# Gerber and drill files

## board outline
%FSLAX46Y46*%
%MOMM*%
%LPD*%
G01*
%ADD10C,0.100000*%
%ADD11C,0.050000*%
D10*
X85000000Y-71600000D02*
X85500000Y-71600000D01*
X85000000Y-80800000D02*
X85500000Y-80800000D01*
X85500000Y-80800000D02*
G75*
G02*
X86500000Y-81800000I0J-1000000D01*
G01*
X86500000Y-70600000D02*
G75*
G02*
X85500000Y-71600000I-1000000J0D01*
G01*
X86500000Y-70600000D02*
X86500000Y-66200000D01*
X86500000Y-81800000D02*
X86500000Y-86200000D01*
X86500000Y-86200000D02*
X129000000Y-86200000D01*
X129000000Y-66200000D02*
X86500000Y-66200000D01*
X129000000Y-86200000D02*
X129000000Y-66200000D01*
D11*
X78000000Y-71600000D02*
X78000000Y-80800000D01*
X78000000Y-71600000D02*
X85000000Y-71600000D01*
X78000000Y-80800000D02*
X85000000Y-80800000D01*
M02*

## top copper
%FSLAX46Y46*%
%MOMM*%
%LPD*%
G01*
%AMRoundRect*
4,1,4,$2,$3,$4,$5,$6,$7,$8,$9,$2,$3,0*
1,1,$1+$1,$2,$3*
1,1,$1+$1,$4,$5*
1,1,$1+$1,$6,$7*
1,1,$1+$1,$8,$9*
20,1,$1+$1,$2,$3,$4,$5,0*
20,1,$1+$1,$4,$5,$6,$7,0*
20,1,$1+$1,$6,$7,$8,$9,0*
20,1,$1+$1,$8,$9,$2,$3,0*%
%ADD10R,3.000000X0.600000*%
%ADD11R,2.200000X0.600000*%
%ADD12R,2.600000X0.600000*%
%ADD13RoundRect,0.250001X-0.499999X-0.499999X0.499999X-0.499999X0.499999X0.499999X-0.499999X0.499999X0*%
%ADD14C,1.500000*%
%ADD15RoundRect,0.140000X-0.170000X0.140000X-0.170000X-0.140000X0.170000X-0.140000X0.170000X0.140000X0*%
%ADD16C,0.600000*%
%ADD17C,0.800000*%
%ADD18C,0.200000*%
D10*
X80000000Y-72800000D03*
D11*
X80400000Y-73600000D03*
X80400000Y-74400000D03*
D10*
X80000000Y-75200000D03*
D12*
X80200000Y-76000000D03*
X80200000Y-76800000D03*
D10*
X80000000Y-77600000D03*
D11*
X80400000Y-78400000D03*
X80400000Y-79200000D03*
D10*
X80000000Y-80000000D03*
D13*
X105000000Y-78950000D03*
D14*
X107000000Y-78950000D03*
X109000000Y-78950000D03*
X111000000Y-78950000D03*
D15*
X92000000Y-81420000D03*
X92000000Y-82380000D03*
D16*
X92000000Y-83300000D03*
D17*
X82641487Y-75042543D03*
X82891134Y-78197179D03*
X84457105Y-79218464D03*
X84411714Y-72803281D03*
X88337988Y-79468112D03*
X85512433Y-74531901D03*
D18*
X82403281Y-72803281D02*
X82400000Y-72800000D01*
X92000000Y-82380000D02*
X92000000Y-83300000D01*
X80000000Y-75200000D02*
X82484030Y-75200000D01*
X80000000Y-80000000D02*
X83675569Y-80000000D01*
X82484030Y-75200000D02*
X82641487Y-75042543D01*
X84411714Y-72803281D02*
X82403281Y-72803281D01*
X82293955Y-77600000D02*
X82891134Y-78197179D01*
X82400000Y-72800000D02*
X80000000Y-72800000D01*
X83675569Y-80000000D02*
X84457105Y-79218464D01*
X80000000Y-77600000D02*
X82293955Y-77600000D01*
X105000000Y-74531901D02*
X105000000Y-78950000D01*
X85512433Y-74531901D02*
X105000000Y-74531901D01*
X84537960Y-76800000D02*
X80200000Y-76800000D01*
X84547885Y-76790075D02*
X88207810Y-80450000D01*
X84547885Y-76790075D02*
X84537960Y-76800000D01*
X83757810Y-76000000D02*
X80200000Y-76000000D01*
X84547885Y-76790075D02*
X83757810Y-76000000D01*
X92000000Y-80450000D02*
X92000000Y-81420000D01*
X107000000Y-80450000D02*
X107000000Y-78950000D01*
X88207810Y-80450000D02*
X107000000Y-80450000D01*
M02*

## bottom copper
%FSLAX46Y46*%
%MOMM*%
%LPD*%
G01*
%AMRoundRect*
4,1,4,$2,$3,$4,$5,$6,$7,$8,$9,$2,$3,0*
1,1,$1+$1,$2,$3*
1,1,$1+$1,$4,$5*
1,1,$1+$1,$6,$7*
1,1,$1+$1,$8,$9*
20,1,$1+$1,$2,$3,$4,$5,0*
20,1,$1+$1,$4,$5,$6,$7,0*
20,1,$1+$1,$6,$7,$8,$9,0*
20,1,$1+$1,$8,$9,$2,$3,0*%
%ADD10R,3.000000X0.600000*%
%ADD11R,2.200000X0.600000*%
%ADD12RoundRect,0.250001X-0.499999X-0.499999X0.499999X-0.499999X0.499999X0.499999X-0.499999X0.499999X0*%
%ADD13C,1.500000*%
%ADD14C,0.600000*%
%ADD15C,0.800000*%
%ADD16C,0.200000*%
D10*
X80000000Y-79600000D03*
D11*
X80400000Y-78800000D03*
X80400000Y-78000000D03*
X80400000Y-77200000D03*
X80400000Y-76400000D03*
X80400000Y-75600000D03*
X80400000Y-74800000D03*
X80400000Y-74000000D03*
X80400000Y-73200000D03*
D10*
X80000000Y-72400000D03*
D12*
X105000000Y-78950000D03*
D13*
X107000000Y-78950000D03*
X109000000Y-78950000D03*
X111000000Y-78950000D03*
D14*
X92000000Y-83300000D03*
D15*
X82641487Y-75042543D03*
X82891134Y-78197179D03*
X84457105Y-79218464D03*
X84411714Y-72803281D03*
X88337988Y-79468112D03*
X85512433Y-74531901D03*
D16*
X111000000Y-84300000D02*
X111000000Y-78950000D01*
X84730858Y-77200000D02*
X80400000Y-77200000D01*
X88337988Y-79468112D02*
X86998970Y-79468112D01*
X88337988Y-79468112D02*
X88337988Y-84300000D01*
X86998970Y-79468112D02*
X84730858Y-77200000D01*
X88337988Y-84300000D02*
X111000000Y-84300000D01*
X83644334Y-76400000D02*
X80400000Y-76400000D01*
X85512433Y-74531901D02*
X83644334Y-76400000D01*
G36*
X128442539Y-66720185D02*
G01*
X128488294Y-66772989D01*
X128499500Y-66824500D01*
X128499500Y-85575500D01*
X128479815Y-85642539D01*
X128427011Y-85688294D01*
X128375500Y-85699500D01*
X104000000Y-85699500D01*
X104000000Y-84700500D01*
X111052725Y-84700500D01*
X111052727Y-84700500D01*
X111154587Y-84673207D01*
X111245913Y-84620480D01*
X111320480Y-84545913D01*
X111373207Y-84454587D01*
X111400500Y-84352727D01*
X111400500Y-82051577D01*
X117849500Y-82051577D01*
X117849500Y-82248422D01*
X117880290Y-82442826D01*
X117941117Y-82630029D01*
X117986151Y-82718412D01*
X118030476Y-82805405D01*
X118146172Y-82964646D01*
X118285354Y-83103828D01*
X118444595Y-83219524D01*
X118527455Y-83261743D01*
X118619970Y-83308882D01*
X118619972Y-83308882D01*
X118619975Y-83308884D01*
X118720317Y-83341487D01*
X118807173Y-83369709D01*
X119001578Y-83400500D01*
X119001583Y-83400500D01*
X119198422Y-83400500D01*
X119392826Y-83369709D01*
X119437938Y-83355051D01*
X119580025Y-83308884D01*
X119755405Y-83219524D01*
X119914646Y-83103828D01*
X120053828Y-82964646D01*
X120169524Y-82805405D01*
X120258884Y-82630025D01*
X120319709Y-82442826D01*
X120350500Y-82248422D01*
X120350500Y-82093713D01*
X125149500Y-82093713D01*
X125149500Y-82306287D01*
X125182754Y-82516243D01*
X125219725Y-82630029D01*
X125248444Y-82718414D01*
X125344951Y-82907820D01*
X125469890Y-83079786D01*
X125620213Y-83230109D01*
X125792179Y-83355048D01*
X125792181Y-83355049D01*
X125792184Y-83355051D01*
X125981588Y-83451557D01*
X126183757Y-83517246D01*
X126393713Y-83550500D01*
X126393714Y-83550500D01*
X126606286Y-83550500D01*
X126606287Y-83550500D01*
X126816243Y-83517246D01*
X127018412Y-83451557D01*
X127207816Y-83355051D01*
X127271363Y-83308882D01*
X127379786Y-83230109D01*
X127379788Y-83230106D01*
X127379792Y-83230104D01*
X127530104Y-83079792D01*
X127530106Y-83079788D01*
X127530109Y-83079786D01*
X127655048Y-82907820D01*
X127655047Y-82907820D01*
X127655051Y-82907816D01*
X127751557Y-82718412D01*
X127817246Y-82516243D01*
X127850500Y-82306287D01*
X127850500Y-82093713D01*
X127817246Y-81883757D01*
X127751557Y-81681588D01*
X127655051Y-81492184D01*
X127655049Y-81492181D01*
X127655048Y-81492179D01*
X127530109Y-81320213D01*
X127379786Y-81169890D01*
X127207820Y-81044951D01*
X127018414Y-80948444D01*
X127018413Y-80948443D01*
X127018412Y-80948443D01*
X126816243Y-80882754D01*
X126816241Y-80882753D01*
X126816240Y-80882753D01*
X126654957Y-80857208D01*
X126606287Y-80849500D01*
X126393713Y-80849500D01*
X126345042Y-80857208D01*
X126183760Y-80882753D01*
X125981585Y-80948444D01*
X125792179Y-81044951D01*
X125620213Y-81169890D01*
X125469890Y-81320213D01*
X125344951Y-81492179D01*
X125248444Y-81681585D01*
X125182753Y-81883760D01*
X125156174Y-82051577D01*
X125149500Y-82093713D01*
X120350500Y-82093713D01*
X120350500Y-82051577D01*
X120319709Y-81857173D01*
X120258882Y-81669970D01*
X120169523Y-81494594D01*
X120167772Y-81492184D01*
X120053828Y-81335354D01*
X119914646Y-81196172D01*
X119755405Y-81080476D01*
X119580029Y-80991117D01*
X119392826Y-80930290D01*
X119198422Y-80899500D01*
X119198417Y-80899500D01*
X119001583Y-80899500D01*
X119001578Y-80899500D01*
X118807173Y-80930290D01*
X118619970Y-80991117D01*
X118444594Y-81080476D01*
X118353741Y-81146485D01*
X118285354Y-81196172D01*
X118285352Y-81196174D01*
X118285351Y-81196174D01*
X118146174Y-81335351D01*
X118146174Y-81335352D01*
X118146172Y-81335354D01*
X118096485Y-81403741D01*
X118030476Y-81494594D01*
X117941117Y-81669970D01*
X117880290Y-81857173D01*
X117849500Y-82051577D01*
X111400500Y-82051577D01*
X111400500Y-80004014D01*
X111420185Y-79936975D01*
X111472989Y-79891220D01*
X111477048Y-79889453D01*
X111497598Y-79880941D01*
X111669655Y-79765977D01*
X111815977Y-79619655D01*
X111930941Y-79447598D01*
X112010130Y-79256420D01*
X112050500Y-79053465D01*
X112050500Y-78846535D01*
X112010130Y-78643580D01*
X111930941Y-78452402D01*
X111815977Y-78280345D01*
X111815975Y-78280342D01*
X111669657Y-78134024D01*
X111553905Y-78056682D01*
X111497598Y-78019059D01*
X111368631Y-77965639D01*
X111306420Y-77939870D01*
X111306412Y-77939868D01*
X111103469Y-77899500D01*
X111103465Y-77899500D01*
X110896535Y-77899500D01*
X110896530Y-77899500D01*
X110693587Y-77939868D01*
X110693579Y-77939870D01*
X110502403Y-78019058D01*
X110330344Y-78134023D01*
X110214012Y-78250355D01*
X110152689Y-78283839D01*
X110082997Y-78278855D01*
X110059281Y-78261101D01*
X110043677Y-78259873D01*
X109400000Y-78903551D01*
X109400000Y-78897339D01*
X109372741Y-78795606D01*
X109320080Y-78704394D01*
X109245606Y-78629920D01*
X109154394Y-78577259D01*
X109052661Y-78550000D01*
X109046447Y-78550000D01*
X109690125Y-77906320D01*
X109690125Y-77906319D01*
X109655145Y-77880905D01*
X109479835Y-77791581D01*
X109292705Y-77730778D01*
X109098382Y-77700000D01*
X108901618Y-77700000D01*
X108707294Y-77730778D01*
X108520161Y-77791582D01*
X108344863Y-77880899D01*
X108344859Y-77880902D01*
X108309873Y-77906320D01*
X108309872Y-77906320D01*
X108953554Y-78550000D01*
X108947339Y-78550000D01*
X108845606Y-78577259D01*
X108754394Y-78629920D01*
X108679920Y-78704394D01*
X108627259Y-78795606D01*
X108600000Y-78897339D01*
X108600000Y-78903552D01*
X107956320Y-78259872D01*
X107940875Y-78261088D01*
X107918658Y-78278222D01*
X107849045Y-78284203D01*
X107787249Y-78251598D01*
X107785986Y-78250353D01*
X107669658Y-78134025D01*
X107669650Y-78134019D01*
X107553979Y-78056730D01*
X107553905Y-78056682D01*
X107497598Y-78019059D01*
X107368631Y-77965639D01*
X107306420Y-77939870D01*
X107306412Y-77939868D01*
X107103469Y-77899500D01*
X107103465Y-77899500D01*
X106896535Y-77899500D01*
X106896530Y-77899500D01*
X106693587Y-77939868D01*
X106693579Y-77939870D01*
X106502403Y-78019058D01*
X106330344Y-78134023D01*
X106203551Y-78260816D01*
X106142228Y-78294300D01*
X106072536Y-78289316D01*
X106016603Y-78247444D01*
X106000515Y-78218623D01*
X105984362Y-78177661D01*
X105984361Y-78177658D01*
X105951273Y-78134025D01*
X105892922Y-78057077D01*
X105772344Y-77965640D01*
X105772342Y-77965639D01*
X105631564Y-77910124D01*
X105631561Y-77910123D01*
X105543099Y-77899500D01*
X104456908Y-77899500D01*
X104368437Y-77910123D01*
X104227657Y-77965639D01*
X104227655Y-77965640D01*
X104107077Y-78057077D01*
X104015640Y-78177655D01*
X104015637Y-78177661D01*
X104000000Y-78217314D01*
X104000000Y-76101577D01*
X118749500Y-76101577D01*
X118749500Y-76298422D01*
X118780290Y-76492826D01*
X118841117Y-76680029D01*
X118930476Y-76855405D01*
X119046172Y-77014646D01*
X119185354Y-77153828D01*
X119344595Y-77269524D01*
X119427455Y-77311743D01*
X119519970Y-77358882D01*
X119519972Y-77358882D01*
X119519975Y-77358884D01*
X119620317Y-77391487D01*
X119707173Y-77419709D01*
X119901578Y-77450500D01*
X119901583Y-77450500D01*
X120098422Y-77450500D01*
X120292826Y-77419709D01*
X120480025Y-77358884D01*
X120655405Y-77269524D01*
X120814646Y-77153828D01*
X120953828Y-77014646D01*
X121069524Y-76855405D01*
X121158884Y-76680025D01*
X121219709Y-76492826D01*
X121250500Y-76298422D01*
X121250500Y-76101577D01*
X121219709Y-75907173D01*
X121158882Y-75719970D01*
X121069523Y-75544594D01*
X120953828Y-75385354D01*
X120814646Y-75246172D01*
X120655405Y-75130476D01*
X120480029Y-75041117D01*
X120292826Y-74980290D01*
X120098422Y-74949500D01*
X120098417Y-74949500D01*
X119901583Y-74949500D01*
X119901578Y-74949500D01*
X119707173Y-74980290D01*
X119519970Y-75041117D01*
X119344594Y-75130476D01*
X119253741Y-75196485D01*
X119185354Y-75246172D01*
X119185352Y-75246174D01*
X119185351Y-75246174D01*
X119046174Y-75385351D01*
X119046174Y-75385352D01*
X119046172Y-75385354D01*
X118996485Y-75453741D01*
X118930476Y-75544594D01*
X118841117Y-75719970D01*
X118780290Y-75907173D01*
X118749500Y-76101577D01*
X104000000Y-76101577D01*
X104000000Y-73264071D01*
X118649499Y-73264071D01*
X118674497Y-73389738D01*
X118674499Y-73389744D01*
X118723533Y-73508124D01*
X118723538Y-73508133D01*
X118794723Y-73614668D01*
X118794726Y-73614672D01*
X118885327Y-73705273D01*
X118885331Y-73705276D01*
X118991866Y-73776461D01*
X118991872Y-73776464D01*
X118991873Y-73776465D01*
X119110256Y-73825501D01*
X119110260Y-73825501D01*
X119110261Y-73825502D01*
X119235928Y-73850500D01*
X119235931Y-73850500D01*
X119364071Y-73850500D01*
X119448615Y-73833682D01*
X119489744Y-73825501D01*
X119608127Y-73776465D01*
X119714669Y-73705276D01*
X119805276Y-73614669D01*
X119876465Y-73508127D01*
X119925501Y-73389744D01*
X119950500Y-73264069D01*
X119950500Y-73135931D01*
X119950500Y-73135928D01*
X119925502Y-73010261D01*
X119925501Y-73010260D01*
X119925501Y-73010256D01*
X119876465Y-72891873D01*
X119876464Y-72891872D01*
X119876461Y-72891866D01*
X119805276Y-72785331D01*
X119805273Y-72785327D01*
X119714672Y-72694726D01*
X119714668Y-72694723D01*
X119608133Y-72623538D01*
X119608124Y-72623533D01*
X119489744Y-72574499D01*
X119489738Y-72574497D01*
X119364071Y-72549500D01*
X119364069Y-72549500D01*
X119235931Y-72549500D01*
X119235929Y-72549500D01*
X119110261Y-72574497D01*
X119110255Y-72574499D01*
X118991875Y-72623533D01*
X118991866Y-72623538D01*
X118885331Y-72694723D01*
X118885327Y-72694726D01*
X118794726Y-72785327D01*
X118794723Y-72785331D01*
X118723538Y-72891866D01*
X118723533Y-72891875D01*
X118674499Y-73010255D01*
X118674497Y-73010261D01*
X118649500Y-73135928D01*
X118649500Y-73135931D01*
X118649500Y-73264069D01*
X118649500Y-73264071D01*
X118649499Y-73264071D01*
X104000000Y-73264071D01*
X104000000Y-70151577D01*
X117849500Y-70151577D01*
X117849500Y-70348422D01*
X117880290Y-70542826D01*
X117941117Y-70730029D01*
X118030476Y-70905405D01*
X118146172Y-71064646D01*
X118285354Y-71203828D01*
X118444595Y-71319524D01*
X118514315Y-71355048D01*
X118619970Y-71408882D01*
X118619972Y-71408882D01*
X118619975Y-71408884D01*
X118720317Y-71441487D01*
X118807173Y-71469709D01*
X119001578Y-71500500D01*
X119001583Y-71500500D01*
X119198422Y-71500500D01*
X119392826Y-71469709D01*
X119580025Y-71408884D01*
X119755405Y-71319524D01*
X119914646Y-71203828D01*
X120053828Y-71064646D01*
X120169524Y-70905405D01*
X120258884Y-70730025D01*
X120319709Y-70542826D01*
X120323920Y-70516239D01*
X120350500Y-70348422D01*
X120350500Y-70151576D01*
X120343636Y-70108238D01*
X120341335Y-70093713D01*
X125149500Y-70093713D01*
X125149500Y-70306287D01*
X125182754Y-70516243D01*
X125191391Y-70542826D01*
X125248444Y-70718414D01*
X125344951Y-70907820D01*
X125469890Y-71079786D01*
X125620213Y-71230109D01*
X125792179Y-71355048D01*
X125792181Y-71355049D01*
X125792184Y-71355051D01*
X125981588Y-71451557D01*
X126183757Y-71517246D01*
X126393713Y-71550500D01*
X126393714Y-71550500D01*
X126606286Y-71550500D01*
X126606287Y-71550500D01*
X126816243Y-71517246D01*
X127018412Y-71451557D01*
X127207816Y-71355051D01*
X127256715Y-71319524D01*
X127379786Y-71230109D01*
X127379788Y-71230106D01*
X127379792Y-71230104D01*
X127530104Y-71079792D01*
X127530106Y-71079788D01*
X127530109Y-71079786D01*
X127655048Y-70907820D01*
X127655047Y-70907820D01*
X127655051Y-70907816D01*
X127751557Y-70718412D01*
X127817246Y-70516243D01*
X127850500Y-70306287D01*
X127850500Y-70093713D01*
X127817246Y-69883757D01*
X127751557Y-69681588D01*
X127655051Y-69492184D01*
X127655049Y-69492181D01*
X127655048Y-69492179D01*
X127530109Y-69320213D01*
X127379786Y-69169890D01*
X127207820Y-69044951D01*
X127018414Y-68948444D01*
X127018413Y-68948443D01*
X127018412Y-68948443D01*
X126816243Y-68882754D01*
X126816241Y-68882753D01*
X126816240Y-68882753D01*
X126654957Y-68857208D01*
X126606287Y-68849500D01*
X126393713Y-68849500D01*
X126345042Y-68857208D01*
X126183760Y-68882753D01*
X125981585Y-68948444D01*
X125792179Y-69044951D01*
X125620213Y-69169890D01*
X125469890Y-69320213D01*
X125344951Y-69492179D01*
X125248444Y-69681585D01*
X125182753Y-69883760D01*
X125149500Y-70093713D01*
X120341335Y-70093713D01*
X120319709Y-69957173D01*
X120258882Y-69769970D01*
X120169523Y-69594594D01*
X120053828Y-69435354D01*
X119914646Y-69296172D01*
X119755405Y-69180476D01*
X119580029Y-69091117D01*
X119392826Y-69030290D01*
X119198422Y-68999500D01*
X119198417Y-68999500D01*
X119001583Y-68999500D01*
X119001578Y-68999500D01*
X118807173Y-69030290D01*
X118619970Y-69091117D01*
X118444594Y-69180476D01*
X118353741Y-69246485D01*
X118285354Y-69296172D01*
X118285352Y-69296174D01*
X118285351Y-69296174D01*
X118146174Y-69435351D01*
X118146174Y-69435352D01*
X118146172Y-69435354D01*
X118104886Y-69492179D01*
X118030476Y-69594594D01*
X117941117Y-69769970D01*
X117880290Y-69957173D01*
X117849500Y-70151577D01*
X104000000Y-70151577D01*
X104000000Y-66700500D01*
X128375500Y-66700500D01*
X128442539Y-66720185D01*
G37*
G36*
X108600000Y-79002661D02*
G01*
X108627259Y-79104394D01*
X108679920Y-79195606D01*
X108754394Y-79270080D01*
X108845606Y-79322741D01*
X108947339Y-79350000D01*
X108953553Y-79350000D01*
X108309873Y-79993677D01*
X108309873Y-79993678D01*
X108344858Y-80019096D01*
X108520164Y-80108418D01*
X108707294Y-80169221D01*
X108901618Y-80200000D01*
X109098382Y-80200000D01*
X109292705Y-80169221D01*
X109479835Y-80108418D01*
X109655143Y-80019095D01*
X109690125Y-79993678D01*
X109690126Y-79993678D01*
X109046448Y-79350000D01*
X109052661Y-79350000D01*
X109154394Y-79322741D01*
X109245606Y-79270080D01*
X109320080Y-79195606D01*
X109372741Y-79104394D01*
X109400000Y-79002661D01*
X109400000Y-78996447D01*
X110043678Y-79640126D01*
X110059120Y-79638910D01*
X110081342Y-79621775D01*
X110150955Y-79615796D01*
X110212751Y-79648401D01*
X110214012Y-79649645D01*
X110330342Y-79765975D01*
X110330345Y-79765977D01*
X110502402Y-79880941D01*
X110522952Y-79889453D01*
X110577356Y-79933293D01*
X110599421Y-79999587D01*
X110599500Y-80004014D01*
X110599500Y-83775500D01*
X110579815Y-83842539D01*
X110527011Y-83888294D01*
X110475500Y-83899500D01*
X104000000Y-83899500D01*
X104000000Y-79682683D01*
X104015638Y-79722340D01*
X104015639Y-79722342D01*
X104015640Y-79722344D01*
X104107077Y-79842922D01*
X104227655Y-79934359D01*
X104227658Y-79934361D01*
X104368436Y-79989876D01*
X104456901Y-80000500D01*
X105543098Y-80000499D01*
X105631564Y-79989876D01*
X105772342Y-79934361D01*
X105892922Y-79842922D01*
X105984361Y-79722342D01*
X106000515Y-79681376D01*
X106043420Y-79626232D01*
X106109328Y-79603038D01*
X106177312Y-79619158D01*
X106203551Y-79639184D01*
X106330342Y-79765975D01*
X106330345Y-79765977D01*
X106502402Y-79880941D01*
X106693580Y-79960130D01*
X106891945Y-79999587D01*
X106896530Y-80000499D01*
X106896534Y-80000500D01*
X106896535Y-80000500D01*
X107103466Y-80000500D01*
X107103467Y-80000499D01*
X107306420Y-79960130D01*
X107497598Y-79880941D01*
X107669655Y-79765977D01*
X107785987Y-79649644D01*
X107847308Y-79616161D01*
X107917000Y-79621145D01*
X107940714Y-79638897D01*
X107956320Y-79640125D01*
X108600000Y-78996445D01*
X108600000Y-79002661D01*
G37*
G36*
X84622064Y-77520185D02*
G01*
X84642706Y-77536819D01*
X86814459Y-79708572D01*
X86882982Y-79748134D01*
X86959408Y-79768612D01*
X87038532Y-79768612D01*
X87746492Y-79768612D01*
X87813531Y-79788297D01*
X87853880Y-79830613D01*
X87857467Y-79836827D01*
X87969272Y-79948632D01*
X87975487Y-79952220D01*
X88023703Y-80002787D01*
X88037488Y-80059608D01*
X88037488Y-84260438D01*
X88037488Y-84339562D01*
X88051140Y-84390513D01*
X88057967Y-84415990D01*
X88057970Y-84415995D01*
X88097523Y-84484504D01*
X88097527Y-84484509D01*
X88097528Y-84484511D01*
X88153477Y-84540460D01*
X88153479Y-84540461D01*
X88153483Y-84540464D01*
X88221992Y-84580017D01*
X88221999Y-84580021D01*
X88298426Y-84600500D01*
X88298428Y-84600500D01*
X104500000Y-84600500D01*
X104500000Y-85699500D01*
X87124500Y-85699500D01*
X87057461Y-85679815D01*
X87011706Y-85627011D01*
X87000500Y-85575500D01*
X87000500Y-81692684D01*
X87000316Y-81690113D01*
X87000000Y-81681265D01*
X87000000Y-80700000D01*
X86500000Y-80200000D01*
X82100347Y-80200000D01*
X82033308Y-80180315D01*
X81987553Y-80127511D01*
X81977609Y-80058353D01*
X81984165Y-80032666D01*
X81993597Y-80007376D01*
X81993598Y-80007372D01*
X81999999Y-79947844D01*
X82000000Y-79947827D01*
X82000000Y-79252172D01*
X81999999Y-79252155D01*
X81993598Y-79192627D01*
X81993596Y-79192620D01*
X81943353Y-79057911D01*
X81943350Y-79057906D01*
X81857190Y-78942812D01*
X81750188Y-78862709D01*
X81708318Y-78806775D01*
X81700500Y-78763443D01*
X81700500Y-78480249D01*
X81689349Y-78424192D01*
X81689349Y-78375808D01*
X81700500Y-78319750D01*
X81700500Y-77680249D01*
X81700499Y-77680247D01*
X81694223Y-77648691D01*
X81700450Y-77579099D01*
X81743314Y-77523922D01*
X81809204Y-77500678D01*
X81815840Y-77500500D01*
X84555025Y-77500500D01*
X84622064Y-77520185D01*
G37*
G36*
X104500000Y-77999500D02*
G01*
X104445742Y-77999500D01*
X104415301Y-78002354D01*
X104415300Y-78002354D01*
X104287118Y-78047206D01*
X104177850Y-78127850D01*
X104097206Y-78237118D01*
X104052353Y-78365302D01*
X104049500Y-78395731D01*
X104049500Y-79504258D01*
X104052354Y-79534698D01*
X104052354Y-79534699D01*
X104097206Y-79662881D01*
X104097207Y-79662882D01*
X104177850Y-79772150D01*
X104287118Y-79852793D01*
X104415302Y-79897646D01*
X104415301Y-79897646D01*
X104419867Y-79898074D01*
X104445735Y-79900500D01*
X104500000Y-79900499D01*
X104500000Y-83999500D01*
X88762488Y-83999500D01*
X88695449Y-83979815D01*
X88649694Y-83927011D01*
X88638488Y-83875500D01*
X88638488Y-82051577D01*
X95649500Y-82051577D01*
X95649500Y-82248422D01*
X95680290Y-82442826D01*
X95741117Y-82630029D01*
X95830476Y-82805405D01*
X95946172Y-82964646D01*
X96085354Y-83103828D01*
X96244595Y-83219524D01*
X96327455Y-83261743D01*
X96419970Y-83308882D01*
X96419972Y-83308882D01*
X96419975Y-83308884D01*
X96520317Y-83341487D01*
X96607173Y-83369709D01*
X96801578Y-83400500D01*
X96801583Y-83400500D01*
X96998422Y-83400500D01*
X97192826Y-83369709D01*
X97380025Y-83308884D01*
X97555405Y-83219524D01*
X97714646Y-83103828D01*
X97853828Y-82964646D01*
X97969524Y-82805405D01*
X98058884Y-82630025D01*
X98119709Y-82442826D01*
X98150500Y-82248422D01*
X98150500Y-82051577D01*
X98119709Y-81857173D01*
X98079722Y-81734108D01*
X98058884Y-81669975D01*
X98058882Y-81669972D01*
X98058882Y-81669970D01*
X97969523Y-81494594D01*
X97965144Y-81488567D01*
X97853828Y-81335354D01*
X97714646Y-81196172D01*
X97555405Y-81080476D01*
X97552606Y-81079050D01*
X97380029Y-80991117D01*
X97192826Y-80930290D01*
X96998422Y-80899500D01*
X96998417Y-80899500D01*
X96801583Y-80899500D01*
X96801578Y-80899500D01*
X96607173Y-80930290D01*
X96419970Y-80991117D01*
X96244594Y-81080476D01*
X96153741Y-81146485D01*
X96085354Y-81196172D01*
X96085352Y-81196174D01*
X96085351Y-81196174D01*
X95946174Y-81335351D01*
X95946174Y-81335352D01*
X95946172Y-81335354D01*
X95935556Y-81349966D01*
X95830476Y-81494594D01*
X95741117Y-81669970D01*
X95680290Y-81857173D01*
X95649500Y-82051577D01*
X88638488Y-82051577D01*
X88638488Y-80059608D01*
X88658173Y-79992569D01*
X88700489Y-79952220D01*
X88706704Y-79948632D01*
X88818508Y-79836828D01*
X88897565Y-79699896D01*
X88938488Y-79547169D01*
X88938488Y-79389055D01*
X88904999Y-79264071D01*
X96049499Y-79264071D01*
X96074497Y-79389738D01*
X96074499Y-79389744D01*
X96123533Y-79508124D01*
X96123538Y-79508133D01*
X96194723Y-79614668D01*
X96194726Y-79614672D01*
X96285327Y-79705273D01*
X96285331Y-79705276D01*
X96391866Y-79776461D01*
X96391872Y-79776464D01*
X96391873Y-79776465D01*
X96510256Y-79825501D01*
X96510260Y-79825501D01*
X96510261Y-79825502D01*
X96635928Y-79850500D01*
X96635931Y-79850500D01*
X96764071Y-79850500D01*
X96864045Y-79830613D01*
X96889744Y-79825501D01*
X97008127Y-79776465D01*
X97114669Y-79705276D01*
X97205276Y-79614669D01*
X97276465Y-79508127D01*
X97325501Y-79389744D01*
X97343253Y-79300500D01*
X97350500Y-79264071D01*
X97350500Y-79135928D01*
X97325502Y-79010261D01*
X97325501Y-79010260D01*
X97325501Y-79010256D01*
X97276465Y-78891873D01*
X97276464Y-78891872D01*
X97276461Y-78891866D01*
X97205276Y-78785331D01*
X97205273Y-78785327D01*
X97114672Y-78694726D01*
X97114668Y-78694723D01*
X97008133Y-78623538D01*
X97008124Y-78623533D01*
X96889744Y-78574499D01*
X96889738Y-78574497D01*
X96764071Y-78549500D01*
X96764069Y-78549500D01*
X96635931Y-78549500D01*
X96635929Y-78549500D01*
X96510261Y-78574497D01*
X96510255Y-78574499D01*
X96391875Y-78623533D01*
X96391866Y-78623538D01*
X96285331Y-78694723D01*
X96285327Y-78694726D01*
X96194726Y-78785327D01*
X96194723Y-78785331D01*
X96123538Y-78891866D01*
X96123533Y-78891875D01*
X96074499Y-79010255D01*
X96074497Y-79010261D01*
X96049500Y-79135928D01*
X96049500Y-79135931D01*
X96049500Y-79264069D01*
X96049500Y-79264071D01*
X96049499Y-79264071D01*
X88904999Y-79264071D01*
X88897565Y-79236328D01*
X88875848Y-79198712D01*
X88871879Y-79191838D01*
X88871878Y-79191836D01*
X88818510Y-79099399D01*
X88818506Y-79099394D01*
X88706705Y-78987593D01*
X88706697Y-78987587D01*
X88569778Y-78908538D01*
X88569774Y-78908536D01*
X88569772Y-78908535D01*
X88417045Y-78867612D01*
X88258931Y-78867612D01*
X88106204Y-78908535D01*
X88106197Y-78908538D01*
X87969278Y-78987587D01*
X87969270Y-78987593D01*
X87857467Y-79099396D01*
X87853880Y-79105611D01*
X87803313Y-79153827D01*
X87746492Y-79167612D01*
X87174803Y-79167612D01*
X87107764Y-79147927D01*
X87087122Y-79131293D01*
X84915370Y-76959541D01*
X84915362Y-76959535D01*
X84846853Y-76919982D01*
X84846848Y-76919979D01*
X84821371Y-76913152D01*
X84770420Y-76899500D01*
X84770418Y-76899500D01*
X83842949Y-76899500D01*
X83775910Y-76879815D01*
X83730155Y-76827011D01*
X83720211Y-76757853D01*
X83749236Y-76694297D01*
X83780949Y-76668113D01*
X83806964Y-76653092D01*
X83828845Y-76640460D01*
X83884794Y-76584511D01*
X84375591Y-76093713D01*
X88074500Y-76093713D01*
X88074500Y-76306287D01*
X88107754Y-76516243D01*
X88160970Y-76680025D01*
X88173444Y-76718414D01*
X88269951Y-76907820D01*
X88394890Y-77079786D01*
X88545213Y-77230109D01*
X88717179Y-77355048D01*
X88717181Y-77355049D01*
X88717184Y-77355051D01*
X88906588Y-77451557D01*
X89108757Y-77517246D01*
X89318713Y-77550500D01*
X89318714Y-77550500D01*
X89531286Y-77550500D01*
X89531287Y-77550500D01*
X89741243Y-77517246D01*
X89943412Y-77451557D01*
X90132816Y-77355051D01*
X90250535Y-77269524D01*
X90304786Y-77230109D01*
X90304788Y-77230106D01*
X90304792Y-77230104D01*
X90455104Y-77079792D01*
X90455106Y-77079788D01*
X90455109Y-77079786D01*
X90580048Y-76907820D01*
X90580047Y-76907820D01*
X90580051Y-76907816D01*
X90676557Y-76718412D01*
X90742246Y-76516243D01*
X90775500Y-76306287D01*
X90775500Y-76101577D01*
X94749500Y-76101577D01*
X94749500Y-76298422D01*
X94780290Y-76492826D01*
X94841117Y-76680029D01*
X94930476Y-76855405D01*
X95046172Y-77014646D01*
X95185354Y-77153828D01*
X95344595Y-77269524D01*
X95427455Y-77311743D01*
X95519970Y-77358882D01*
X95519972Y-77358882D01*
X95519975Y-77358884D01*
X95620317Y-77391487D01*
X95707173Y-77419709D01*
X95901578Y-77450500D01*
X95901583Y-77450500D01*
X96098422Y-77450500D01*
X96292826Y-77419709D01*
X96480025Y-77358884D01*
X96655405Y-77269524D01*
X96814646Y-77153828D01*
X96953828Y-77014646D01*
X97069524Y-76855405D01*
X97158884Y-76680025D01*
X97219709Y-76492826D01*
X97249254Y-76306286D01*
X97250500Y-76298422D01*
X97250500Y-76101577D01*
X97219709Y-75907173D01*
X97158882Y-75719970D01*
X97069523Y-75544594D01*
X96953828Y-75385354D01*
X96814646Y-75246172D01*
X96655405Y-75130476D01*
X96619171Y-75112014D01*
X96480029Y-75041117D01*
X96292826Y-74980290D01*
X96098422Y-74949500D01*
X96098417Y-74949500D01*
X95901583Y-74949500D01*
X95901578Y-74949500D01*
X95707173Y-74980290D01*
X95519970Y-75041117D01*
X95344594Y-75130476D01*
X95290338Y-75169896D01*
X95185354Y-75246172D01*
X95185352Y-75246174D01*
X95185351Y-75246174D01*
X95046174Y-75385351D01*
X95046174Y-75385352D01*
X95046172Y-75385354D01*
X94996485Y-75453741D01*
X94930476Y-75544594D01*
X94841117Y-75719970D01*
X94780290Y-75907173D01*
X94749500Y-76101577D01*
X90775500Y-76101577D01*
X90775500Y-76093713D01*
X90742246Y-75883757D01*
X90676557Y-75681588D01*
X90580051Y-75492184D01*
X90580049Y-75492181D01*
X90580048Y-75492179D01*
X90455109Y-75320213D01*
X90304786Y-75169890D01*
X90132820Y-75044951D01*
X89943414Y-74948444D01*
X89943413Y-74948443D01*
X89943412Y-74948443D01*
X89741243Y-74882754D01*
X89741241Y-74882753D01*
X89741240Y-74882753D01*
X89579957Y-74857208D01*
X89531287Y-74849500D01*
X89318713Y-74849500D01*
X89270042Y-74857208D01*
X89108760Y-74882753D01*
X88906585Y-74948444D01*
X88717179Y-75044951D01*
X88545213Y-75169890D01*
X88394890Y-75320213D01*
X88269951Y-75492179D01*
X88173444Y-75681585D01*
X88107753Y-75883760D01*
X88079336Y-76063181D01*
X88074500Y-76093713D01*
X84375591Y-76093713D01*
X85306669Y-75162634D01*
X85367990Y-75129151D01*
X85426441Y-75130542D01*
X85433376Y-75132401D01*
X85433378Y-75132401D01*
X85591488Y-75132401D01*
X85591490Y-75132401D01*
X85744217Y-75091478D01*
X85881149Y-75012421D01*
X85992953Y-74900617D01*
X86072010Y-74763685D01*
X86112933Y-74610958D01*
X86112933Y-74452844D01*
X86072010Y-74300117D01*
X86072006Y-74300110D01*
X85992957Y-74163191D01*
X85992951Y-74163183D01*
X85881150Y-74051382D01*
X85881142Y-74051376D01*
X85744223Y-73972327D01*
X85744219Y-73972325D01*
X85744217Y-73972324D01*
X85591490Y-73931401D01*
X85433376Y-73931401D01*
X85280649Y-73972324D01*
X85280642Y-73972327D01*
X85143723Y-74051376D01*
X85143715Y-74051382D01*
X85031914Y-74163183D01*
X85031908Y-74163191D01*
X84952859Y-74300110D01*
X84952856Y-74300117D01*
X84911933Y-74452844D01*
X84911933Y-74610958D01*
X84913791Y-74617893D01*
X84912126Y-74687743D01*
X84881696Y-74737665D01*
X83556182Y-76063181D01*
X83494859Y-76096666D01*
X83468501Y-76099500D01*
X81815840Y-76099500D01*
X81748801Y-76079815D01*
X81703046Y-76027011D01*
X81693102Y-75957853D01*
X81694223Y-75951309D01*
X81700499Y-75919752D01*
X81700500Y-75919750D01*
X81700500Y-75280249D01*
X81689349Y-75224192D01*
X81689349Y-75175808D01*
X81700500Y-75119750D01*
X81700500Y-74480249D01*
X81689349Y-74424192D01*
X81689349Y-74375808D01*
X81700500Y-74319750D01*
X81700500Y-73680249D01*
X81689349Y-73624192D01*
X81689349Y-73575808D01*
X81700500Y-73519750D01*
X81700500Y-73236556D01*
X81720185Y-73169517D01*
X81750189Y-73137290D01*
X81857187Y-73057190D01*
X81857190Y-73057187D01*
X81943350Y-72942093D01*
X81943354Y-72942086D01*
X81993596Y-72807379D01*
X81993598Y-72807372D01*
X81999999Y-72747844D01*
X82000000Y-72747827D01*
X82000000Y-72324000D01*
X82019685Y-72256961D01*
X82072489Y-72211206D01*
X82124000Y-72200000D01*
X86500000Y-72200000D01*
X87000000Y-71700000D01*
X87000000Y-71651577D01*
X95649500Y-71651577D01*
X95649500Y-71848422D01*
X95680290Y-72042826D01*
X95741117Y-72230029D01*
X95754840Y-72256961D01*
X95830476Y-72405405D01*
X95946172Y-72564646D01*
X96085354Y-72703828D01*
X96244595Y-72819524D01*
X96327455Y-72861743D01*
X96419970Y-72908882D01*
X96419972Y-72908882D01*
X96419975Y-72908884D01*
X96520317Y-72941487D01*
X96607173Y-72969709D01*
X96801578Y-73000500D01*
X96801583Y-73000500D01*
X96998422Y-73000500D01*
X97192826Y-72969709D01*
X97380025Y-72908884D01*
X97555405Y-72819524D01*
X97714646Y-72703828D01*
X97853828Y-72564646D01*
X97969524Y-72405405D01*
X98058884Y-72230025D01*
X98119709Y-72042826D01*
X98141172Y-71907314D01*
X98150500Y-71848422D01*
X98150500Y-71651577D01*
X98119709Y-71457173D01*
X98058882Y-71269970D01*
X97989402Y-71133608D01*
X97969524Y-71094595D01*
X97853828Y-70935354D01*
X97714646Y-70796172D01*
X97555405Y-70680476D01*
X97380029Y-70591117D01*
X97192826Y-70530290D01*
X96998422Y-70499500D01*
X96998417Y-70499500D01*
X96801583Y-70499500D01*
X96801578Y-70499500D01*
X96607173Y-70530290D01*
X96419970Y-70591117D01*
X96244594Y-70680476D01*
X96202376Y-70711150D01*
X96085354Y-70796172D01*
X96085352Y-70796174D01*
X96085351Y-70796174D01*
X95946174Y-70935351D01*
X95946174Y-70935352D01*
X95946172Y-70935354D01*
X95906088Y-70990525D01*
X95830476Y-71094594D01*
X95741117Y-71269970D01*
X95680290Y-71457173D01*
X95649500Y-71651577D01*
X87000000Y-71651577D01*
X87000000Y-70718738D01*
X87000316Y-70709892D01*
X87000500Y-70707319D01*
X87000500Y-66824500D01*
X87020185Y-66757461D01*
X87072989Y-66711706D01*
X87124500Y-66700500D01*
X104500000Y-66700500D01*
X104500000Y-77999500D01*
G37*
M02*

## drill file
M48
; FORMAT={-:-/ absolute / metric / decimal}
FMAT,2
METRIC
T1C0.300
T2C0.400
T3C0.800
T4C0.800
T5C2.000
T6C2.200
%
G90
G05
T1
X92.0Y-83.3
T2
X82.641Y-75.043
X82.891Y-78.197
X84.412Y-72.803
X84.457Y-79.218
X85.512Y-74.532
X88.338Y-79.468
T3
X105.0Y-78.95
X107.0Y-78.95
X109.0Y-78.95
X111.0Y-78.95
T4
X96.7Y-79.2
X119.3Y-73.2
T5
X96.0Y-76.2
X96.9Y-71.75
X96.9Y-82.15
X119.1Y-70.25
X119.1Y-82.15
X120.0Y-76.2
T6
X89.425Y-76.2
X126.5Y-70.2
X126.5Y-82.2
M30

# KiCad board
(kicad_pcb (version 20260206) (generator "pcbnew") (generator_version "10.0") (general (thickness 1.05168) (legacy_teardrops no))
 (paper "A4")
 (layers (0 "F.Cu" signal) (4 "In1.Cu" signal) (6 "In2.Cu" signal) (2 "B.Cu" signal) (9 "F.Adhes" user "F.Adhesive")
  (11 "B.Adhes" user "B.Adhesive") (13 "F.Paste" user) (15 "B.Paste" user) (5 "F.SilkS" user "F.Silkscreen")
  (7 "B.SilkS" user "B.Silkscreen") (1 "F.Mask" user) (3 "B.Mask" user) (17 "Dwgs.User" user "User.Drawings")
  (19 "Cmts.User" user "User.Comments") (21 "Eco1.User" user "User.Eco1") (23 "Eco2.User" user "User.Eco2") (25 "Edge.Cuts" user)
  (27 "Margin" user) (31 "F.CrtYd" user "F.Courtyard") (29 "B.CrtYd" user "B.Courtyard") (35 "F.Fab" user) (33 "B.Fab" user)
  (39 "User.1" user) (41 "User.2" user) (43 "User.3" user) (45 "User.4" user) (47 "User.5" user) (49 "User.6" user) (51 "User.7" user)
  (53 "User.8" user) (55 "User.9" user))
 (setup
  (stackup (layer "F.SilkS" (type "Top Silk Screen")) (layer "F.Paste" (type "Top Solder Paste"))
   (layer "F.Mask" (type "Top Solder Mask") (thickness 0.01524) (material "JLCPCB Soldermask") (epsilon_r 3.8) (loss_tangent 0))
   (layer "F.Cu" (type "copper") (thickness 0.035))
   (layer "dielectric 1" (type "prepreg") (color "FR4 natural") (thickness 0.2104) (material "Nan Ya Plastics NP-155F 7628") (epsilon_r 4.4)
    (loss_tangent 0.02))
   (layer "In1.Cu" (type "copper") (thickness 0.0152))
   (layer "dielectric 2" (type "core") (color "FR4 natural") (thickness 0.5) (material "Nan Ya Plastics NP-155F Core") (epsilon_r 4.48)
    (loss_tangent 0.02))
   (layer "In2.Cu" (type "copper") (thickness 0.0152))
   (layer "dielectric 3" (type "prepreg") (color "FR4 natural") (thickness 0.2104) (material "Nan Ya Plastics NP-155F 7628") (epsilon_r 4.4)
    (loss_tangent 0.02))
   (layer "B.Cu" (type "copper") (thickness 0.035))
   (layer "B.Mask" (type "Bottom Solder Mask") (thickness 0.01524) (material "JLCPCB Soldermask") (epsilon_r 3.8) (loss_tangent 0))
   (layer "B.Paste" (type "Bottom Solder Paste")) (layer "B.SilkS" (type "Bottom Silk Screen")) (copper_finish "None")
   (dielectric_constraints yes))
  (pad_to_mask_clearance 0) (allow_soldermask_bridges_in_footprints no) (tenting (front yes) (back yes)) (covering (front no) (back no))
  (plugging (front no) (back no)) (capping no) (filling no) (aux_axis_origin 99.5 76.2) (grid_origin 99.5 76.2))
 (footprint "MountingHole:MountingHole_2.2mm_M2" (layer "F.Cu") (at 126.5 82.2)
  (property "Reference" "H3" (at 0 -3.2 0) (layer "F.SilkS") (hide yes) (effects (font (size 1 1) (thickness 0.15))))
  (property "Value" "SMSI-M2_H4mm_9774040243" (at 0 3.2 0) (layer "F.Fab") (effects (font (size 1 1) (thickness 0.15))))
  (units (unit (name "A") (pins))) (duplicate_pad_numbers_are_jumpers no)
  (pad "" np_thru_hole circle (at 0 0) (size 2.2 2.2) (drill 2.2) (layers "*.Cu" "*.Mask")))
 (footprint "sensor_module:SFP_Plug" (layer "F.Cu") (at 81.5 76.2 180)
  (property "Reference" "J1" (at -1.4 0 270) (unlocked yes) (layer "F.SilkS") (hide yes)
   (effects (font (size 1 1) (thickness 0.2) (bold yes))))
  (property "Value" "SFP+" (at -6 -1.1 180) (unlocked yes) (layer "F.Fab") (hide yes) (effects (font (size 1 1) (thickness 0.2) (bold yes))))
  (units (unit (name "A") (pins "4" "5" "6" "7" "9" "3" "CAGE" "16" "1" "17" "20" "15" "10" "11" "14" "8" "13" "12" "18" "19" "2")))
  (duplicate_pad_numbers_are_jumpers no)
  (fp_line (start 3.5 4.6) (end 3.5 -4.6) (stroke (width 0.05) (type default)) (layer "Edge.Cuts"))
  (fp_line (start 3.5 4.6) (end -3.5 4.6) (stroke (width 0.05) (type solid)) (layer "Edge.Cuts"))
  (fp_line (start 3.5 -4.6) (end -3.5 -4.6) (stroke (width 0.05) (type solid)) (layer "Edge.Cuts"))
  (pad "1" smd rect (at 1.5 -3.4 180) (size 3 0.6) (layers "B.Cu" "B.Mask") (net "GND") (thermal_bridge_angle 45))
  (pad "2" smd rect (at 1.1 -2.6 180) (size 2.2 0.6) (layers "B.Cu" "B.Mask") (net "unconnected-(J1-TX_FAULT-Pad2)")
   (thermal_bridge_angle 45))
  (pad "3" smd rect (at 1.1 -1.8 180) (size 2.2 0.6) (layers "B.Cu" "B.Mask") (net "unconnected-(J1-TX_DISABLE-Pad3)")
   (thermal_bridge_angle 45))
  (pad "4" smd rect (at 1.1 -1 180) (size 2.2 0.6) (layers "B.Cu" "B.Mask") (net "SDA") (thermal_bridge_angle 45))
  (pad "5" smd rect (at 1.1 -0.2 180) (size 2.2 0.6) (layers "B.Cu" "B.Mask") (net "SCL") (thermal_bridge_angle 45))
  (pad "6" smd rect (at 1.1 0.6 180) (size 2.2 0.6) (layers "B.Cu" "B.Mask") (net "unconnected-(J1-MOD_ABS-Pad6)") (thermal_bridge_angle 45))
  (pad "7" smd rect (at 1.1 1.4 180) (size 2.2 0.6) (layers "B.Cu" "B.Mask") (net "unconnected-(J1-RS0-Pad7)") (thermal_bridge_angle 45))
  (pad "8" smd rect (at 1.1 2.2 180) (size 2.2 0.6) (layers "B.Cu" "B.Mask") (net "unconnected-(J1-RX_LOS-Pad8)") (thermal_bridge_angle 45))
  (pad "9" smd rect (at 1.1 3 180) (size 2.2 0.6) (layers "B.Cu" "B.Mask") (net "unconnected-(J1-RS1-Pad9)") (thermal_bridge_angle 45))
  (pad "10" smd rect (at 1.5 3.8 180) (size 3 0.6) (layers "B.Cu" "B.Mask") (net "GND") (thermal_bridge_angle 45))
  (pad "11" smd rect (at 1.5 3.4 180) (size 3 0.6) (layers "F.Cu" "F.Mask") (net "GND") (thermal_bridge_angle 45))
  (pad "12" smd rect (at 1.1 2.6 180) (size 2.2 0.6) (layers "F.Cu" "F.Mask") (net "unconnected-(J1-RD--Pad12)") (thermal_bridge_angle 45))
  (pad "13" smd rect (at 1.1 1.8 180) (size 2.2 0.6) (layers "F.Cu" "F.Mask") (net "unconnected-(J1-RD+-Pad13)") (thermal_bridge_angle 45))
  (pad "14" smd rect (at 1.5 1 180) (size 3 0.6) (layers "F.Cu" "F.Mask") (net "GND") (thermal_bridge_angle 45))
  (pad "15" smd rect (at 1.3 0.2 180) (size 2.6 0.6) (layers "F.Cu" "F.Mask") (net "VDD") (thermal_bridge_angle 45))
  (pad "16" smd rect (at 1.3 -0.6 180) (size 2.6 0.6) (layers "F.Cu" "F.Mask") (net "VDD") (thermal_bridge_angle 45))
  (pad "17" smd rect (at 1.5 -1.4 180) (size 3 0.6) (layers "F.Cu" "F.Mask") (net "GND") (thermal_bridge_angle 45))
  (pad "18" smd rect (at 1.1 -2.2 180) (size 2.2 0.6) (layers "F.Cu" "F.Mask") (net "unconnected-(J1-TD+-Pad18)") (thermal_bridge_angle 45))
  (pad "19" smd rect (at 1.1 -3 180) (size 2.2 0.6) (layers "F.Cu" "F.Mask") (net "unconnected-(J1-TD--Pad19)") (thermal_bridge_angle 45))
  (pad "20" smd rect (at 1.5 -3.8 180) (size 3 0.6) (layers "F.Cu" "F.Mask") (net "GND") (thermal_bridge_angle 45)))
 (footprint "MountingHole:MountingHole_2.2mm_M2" (layer "F.Cu") (at 126.5 70.2)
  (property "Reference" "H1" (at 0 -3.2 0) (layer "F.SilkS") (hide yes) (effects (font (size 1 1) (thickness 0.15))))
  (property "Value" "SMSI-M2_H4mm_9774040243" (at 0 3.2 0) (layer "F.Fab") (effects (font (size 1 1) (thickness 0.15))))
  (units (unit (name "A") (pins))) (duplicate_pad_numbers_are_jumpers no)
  (pad "" np_thru_hole circle (at 0 0) (size 2.2 2.2) (drill 2.2) (layers "*.Cu" "*.Mask")))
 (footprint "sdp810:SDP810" (layer "F.Cu") (at 108 76.2)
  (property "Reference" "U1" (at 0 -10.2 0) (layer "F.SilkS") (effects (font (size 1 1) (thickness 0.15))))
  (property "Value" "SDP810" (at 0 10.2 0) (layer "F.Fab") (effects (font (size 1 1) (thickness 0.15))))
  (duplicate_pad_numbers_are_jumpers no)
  (pad "" np_thru_hole circle (at -12 0) (size 2 2) (drill 2) (layers "*.Cu" "*.Mask"))
  (pad "" np_thru_hole circle (at -11.3 3) (size 0.8 0.8) (drill 0.8) (layers "*.Cu" "*.Mask"))
  (pad "" np_thru_hole circle (at -11.1 -4.45) (size 2 2) (drill 2) (layers "*.Cu" "*.Mask"))
  (pad "" np_thru_hole circle (at -11.1 5.95) (size 2 2) (drill 2) (layers "*.Cu" "*.Mask"))
  (pad "" np_thru_hole circle (at 11.1 -5.95) (size 2 2) (drill 2) (layers "*.Cu" "*.Mask"))
  (pad "" np_thru_hole circle (at 11.1 5.95) (size 2 2) (drill 2) (layers "*.Cu" "*.Mask"))
  (pad "" np_thru_hole circle (at 11.3 -3) (size 0.8 0.8) (drill 0.8) (layers "*.Cu" "*.Mask"))
  (pad "" np_thru_hole circle (at 12 0) (size 2 2) (drill 2) (layers "*.Cu" "*.Mask"))
  (pad "1" thru_hole roundrect (at -3 2.75) (size 1.5 1.5) (drill 0.8) (layers "*.Cu" "*.Mask") (remove_unused_layers no)
   (roundrect_rratio 0.166667) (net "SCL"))
  (pad "2" thru_hole circle (at -1 2.75) (size 1.5 1.5) (drill 0.8) (layers "*.Cu" "*.Mask") (remove_unused_layers no) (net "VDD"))
  (pad "3" thru_hole circle (at 1 2.75) (size 1.5 1.5) (drill 0.8) (layers "*.Cu" "*.Mask") (remove_unused_layers no) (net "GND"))
  (pad "4" thru_hole circle (at 3 2.75) (size 1.5 1.5) (drill 0.8) (layers "*.Cu" "*.Mask") (remove_unused_layers no) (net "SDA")))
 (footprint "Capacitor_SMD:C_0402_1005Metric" (layer "F.Cu") (at 92 81.9 -90)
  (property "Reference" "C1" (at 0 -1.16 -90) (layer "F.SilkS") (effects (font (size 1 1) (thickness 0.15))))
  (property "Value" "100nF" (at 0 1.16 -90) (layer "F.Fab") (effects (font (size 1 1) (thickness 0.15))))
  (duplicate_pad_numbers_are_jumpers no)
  (pad "1" smd roundrect (at -0.48 0 270) (size 0.56 0.62) (layers "F.Cu" "F.Mask" "F.Paste") (roundrect_rratio 0.25) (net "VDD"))
  (pad "2" smd roundrect (at 0.48 0 270) (size 0.56 0.62) (layers "F.Cu" "F.Mask" "F.Paste") (roundrect_rratio 0.25) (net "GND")))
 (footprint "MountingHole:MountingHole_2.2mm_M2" (layer "F.Cu") (at 89.425 76.2)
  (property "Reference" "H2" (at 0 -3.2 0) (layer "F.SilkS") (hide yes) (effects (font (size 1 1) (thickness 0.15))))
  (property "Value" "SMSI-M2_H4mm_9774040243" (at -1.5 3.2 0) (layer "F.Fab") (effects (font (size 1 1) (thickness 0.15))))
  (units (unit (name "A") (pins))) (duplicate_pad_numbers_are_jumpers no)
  (pad "" np_thru_hole circle (at 0 0) (size 2.2 2.2) (drill 2.2) (layers "*.Cu" "*.Mask")))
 (gr_line (start 85 71.6) (end 85.5 71.6) (stroke (width 0.1) (type default)) (layer "Edge.Cuts"))
 (gr_line (start 85 80.8) (end 85.5 80.8) (stroke (width 0.1) (type default)) (layer "Edge.Cuts"))
 (gr_arc (start 85.5 80.8) (mid 86.207107 81.092893) (end 86.5 81.8) (stroke (width 0.1) (type default)) (layer "Edge.Cuts"))
 (gr_arc (start 86.5 70.6) (mid 86.207107 71.307107) (end 85.5 71.6) (stroke (width 0.1) (type default)) (layer "Edge.Cuts"))
 (gr_line (start 86.5 70.6) (end 86.5 66.2) (stroke (width 0.1) (type default)) (layer "Edge.Cuts"))
 (gr_line (start 86.5 81.8) (end 86.5 86.2) (stroke (width 0.1) (type default)) (layer "Edge.Cuts"))
 (gr_line (start 86.5 86.2) (end 129 86.2) (stroke (width 0.1) (type default)) (layer "Edge.Cuts"))
 (gr_line (start 129 66.2) (end 86.5 66.2) (stroke (width 0.1) (type default)) (layer "Edge.Cuts"))
 (gr_line (start 129 86.2) (end 129 66.2) (stroke (width 0.1) (type default)) (layer "Edge.Cuts"))
 (segment (start 82.403281 72.803281) (end 82.4 72.8) (width 0.2) (layer "F.Cu") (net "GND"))
 (segment (start 92 82.38) (end 92 83.3) (width 0.2) (layer "F.Cu") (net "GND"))
 (segment (start 80 75.2) (end 82.48403 75.2) (width 0.2) (layer "F.Cu") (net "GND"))
 (segment (start 80 80) (end 83.675569 80) (width 0.2) (layer "F.Cu") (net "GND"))
 (segment (start 82.48403 75.2) (end 82.641487 75.042543) (width 0.2) (layer "F.Cu") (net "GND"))
 (segment (start 84.411714 72.803281) (end 82.403281 72.803281) (width 0.2) (layer "F.Cu") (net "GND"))
 (segment (start 82.293955 77.6) (end 82.891134 78.197179) (width 0.2) (layer "F.Cu") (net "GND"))
 (segment (start 82.4 72.8) (end 80 72.8) (width 0.2) (layer "F.Cu") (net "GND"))
 (segment (start 83.675569 80) (end 84.457105 79.218464) (width 0.2) (layer "F.Cu") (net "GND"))
 (segment (start 80 77.6) (end 82.293955 77.6) (width 0.2) (layer "F.Cu") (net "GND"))
 (via (at 92 83.3) (size 0.6) (drill 0.3) (layers "F.Cu" "B.Cu") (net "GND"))
 (via (at 82.641487 75.042543) (size 0.8) (drill 0.4) (layers "F.Cu" "B.Cu") (capping no) (covering (front no) (back no))
  (plugging (front no) (back no)) (filling no) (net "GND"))
 (via (at 82.891134 78.197179) (size 0.8) (drill 0.4) (layers "F.Cu" "B.Cu") (capping no) (covering (front no) (back no))
  (plugging (front no) (back no)) (filling no) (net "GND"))
 (via (at 84.457105 79.218464) (size 0.8) (drill 0.4) (layers "F.Cu" "B.Cu") (capping no) (covering (front no) (back no))
  (plugging (front no) (back no)) (filling no) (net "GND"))
 (via (at 84.411714 72.803281) (size 0.8) (drill 0.4) (layers "F.Cu" "B.Cu") (capping no) (covering (front no) (back no))
  (plugging (front no) (back no)) (filling no) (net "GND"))
 (via (at 88.337988 79.468112) (size 0.8) (drill 0.4) (layers "F.Cu" "B.Cu") (capping no) (covering (front no) (back no))
  (plugging (front no) (back no)) (filling no) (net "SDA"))
 (segment (start 111 84.3) (end 111 78.95) (width 0.2) (layer "B.Cu") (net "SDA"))
 (segment (start 84.730858 77.2) (end 80.4 77.2) (width 0.2) (layer "B.Cu") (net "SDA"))
 (segment (start 88.337988 79.468112) (end 86.99897 79.468112) (width 0.2) (layer "B.Cu") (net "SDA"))
 (segment (start 88.337988 79.468112) (end 88.337988 84.3) (width 0.2) (layer "B.Cu") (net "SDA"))
 (segment (start 86.99897 79.468112) (end 84.730858 77.2) (width 0.2) (layer "B.Cu") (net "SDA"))
 (segment (start 88.337988 84.3) (end 111 84.3) (width 0.2) (layer "B.Cu") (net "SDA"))
 (segment (start 105 74.531901) (end 105 78.95) (width 0.2) (layer "F.Cu") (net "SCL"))
 (segment (start 85.512433 74.531901) (end 105 74.531901) (width 0.2) (layer "F.Cu") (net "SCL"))
 (via (at 85.512433 74.531901) (size 0.8) (drill 0.4) (layers "F.Cu" "B.Cu") (capping no) (covering (front no) (back no))
  (plugging (front no) (back no)) (filling no) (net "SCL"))
 (segment (start 83.644334 76.4) (end 80.4 76.4) (width 0.2) (layer "B.Cu") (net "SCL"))
 (segment (start 85.512433 74.531901) (end 83.644334 76.4) (width 0.2) (layer "B.Cu") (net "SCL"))
 (segment (start 84.53796 76.8) (end 80.2 76.8) (width 0.2) (layer "F.Cu") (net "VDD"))
 (segment (start 84.547885 76.790075) (end 88.20781 80.45) (width 0.2) (layer "F.Cu") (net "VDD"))
 (segment (start 84.547885 76.790075) (end 84.53796 76.8) (width 0.2) (layer "F.Cu") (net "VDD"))
 (segment (start 83.75781 76) (end 80.2 76) (width 0.2) (layer "F.Cu") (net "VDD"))
 (segment (start 84.547885 76.790075) (end 83.75781 76) (width 0.2) (layer "F.Cu") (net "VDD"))
 (segment (start 92 80.45) (end 92 81.42) (width 0.2) (layer "F.Cu") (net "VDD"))
 (segment (start 107 80.45) (end 107 78.95) (width 0.2) (layer "F.Cu") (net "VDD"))
 (segment (start 88.20781 80.45) (end 107 80.45) (width 0.2) (layer "F.Cu") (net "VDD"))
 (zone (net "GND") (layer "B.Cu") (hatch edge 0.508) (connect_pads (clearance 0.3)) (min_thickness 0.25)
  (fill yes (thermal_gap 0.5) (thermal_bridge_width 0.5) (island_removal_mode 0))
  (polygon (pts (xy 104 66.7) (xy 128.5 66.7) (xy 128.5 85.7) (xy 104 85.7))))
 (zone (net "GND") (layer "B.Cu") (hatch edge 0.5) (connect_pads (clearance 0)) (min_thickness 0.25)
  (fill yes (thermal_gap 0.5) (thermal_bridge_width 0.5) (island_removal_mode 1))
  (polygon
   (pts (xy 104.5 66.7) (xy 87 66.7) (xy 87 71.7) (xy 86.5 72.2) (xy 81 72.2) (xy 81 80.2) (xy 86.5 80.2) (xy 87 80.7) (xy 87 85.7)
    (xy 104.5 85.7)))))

